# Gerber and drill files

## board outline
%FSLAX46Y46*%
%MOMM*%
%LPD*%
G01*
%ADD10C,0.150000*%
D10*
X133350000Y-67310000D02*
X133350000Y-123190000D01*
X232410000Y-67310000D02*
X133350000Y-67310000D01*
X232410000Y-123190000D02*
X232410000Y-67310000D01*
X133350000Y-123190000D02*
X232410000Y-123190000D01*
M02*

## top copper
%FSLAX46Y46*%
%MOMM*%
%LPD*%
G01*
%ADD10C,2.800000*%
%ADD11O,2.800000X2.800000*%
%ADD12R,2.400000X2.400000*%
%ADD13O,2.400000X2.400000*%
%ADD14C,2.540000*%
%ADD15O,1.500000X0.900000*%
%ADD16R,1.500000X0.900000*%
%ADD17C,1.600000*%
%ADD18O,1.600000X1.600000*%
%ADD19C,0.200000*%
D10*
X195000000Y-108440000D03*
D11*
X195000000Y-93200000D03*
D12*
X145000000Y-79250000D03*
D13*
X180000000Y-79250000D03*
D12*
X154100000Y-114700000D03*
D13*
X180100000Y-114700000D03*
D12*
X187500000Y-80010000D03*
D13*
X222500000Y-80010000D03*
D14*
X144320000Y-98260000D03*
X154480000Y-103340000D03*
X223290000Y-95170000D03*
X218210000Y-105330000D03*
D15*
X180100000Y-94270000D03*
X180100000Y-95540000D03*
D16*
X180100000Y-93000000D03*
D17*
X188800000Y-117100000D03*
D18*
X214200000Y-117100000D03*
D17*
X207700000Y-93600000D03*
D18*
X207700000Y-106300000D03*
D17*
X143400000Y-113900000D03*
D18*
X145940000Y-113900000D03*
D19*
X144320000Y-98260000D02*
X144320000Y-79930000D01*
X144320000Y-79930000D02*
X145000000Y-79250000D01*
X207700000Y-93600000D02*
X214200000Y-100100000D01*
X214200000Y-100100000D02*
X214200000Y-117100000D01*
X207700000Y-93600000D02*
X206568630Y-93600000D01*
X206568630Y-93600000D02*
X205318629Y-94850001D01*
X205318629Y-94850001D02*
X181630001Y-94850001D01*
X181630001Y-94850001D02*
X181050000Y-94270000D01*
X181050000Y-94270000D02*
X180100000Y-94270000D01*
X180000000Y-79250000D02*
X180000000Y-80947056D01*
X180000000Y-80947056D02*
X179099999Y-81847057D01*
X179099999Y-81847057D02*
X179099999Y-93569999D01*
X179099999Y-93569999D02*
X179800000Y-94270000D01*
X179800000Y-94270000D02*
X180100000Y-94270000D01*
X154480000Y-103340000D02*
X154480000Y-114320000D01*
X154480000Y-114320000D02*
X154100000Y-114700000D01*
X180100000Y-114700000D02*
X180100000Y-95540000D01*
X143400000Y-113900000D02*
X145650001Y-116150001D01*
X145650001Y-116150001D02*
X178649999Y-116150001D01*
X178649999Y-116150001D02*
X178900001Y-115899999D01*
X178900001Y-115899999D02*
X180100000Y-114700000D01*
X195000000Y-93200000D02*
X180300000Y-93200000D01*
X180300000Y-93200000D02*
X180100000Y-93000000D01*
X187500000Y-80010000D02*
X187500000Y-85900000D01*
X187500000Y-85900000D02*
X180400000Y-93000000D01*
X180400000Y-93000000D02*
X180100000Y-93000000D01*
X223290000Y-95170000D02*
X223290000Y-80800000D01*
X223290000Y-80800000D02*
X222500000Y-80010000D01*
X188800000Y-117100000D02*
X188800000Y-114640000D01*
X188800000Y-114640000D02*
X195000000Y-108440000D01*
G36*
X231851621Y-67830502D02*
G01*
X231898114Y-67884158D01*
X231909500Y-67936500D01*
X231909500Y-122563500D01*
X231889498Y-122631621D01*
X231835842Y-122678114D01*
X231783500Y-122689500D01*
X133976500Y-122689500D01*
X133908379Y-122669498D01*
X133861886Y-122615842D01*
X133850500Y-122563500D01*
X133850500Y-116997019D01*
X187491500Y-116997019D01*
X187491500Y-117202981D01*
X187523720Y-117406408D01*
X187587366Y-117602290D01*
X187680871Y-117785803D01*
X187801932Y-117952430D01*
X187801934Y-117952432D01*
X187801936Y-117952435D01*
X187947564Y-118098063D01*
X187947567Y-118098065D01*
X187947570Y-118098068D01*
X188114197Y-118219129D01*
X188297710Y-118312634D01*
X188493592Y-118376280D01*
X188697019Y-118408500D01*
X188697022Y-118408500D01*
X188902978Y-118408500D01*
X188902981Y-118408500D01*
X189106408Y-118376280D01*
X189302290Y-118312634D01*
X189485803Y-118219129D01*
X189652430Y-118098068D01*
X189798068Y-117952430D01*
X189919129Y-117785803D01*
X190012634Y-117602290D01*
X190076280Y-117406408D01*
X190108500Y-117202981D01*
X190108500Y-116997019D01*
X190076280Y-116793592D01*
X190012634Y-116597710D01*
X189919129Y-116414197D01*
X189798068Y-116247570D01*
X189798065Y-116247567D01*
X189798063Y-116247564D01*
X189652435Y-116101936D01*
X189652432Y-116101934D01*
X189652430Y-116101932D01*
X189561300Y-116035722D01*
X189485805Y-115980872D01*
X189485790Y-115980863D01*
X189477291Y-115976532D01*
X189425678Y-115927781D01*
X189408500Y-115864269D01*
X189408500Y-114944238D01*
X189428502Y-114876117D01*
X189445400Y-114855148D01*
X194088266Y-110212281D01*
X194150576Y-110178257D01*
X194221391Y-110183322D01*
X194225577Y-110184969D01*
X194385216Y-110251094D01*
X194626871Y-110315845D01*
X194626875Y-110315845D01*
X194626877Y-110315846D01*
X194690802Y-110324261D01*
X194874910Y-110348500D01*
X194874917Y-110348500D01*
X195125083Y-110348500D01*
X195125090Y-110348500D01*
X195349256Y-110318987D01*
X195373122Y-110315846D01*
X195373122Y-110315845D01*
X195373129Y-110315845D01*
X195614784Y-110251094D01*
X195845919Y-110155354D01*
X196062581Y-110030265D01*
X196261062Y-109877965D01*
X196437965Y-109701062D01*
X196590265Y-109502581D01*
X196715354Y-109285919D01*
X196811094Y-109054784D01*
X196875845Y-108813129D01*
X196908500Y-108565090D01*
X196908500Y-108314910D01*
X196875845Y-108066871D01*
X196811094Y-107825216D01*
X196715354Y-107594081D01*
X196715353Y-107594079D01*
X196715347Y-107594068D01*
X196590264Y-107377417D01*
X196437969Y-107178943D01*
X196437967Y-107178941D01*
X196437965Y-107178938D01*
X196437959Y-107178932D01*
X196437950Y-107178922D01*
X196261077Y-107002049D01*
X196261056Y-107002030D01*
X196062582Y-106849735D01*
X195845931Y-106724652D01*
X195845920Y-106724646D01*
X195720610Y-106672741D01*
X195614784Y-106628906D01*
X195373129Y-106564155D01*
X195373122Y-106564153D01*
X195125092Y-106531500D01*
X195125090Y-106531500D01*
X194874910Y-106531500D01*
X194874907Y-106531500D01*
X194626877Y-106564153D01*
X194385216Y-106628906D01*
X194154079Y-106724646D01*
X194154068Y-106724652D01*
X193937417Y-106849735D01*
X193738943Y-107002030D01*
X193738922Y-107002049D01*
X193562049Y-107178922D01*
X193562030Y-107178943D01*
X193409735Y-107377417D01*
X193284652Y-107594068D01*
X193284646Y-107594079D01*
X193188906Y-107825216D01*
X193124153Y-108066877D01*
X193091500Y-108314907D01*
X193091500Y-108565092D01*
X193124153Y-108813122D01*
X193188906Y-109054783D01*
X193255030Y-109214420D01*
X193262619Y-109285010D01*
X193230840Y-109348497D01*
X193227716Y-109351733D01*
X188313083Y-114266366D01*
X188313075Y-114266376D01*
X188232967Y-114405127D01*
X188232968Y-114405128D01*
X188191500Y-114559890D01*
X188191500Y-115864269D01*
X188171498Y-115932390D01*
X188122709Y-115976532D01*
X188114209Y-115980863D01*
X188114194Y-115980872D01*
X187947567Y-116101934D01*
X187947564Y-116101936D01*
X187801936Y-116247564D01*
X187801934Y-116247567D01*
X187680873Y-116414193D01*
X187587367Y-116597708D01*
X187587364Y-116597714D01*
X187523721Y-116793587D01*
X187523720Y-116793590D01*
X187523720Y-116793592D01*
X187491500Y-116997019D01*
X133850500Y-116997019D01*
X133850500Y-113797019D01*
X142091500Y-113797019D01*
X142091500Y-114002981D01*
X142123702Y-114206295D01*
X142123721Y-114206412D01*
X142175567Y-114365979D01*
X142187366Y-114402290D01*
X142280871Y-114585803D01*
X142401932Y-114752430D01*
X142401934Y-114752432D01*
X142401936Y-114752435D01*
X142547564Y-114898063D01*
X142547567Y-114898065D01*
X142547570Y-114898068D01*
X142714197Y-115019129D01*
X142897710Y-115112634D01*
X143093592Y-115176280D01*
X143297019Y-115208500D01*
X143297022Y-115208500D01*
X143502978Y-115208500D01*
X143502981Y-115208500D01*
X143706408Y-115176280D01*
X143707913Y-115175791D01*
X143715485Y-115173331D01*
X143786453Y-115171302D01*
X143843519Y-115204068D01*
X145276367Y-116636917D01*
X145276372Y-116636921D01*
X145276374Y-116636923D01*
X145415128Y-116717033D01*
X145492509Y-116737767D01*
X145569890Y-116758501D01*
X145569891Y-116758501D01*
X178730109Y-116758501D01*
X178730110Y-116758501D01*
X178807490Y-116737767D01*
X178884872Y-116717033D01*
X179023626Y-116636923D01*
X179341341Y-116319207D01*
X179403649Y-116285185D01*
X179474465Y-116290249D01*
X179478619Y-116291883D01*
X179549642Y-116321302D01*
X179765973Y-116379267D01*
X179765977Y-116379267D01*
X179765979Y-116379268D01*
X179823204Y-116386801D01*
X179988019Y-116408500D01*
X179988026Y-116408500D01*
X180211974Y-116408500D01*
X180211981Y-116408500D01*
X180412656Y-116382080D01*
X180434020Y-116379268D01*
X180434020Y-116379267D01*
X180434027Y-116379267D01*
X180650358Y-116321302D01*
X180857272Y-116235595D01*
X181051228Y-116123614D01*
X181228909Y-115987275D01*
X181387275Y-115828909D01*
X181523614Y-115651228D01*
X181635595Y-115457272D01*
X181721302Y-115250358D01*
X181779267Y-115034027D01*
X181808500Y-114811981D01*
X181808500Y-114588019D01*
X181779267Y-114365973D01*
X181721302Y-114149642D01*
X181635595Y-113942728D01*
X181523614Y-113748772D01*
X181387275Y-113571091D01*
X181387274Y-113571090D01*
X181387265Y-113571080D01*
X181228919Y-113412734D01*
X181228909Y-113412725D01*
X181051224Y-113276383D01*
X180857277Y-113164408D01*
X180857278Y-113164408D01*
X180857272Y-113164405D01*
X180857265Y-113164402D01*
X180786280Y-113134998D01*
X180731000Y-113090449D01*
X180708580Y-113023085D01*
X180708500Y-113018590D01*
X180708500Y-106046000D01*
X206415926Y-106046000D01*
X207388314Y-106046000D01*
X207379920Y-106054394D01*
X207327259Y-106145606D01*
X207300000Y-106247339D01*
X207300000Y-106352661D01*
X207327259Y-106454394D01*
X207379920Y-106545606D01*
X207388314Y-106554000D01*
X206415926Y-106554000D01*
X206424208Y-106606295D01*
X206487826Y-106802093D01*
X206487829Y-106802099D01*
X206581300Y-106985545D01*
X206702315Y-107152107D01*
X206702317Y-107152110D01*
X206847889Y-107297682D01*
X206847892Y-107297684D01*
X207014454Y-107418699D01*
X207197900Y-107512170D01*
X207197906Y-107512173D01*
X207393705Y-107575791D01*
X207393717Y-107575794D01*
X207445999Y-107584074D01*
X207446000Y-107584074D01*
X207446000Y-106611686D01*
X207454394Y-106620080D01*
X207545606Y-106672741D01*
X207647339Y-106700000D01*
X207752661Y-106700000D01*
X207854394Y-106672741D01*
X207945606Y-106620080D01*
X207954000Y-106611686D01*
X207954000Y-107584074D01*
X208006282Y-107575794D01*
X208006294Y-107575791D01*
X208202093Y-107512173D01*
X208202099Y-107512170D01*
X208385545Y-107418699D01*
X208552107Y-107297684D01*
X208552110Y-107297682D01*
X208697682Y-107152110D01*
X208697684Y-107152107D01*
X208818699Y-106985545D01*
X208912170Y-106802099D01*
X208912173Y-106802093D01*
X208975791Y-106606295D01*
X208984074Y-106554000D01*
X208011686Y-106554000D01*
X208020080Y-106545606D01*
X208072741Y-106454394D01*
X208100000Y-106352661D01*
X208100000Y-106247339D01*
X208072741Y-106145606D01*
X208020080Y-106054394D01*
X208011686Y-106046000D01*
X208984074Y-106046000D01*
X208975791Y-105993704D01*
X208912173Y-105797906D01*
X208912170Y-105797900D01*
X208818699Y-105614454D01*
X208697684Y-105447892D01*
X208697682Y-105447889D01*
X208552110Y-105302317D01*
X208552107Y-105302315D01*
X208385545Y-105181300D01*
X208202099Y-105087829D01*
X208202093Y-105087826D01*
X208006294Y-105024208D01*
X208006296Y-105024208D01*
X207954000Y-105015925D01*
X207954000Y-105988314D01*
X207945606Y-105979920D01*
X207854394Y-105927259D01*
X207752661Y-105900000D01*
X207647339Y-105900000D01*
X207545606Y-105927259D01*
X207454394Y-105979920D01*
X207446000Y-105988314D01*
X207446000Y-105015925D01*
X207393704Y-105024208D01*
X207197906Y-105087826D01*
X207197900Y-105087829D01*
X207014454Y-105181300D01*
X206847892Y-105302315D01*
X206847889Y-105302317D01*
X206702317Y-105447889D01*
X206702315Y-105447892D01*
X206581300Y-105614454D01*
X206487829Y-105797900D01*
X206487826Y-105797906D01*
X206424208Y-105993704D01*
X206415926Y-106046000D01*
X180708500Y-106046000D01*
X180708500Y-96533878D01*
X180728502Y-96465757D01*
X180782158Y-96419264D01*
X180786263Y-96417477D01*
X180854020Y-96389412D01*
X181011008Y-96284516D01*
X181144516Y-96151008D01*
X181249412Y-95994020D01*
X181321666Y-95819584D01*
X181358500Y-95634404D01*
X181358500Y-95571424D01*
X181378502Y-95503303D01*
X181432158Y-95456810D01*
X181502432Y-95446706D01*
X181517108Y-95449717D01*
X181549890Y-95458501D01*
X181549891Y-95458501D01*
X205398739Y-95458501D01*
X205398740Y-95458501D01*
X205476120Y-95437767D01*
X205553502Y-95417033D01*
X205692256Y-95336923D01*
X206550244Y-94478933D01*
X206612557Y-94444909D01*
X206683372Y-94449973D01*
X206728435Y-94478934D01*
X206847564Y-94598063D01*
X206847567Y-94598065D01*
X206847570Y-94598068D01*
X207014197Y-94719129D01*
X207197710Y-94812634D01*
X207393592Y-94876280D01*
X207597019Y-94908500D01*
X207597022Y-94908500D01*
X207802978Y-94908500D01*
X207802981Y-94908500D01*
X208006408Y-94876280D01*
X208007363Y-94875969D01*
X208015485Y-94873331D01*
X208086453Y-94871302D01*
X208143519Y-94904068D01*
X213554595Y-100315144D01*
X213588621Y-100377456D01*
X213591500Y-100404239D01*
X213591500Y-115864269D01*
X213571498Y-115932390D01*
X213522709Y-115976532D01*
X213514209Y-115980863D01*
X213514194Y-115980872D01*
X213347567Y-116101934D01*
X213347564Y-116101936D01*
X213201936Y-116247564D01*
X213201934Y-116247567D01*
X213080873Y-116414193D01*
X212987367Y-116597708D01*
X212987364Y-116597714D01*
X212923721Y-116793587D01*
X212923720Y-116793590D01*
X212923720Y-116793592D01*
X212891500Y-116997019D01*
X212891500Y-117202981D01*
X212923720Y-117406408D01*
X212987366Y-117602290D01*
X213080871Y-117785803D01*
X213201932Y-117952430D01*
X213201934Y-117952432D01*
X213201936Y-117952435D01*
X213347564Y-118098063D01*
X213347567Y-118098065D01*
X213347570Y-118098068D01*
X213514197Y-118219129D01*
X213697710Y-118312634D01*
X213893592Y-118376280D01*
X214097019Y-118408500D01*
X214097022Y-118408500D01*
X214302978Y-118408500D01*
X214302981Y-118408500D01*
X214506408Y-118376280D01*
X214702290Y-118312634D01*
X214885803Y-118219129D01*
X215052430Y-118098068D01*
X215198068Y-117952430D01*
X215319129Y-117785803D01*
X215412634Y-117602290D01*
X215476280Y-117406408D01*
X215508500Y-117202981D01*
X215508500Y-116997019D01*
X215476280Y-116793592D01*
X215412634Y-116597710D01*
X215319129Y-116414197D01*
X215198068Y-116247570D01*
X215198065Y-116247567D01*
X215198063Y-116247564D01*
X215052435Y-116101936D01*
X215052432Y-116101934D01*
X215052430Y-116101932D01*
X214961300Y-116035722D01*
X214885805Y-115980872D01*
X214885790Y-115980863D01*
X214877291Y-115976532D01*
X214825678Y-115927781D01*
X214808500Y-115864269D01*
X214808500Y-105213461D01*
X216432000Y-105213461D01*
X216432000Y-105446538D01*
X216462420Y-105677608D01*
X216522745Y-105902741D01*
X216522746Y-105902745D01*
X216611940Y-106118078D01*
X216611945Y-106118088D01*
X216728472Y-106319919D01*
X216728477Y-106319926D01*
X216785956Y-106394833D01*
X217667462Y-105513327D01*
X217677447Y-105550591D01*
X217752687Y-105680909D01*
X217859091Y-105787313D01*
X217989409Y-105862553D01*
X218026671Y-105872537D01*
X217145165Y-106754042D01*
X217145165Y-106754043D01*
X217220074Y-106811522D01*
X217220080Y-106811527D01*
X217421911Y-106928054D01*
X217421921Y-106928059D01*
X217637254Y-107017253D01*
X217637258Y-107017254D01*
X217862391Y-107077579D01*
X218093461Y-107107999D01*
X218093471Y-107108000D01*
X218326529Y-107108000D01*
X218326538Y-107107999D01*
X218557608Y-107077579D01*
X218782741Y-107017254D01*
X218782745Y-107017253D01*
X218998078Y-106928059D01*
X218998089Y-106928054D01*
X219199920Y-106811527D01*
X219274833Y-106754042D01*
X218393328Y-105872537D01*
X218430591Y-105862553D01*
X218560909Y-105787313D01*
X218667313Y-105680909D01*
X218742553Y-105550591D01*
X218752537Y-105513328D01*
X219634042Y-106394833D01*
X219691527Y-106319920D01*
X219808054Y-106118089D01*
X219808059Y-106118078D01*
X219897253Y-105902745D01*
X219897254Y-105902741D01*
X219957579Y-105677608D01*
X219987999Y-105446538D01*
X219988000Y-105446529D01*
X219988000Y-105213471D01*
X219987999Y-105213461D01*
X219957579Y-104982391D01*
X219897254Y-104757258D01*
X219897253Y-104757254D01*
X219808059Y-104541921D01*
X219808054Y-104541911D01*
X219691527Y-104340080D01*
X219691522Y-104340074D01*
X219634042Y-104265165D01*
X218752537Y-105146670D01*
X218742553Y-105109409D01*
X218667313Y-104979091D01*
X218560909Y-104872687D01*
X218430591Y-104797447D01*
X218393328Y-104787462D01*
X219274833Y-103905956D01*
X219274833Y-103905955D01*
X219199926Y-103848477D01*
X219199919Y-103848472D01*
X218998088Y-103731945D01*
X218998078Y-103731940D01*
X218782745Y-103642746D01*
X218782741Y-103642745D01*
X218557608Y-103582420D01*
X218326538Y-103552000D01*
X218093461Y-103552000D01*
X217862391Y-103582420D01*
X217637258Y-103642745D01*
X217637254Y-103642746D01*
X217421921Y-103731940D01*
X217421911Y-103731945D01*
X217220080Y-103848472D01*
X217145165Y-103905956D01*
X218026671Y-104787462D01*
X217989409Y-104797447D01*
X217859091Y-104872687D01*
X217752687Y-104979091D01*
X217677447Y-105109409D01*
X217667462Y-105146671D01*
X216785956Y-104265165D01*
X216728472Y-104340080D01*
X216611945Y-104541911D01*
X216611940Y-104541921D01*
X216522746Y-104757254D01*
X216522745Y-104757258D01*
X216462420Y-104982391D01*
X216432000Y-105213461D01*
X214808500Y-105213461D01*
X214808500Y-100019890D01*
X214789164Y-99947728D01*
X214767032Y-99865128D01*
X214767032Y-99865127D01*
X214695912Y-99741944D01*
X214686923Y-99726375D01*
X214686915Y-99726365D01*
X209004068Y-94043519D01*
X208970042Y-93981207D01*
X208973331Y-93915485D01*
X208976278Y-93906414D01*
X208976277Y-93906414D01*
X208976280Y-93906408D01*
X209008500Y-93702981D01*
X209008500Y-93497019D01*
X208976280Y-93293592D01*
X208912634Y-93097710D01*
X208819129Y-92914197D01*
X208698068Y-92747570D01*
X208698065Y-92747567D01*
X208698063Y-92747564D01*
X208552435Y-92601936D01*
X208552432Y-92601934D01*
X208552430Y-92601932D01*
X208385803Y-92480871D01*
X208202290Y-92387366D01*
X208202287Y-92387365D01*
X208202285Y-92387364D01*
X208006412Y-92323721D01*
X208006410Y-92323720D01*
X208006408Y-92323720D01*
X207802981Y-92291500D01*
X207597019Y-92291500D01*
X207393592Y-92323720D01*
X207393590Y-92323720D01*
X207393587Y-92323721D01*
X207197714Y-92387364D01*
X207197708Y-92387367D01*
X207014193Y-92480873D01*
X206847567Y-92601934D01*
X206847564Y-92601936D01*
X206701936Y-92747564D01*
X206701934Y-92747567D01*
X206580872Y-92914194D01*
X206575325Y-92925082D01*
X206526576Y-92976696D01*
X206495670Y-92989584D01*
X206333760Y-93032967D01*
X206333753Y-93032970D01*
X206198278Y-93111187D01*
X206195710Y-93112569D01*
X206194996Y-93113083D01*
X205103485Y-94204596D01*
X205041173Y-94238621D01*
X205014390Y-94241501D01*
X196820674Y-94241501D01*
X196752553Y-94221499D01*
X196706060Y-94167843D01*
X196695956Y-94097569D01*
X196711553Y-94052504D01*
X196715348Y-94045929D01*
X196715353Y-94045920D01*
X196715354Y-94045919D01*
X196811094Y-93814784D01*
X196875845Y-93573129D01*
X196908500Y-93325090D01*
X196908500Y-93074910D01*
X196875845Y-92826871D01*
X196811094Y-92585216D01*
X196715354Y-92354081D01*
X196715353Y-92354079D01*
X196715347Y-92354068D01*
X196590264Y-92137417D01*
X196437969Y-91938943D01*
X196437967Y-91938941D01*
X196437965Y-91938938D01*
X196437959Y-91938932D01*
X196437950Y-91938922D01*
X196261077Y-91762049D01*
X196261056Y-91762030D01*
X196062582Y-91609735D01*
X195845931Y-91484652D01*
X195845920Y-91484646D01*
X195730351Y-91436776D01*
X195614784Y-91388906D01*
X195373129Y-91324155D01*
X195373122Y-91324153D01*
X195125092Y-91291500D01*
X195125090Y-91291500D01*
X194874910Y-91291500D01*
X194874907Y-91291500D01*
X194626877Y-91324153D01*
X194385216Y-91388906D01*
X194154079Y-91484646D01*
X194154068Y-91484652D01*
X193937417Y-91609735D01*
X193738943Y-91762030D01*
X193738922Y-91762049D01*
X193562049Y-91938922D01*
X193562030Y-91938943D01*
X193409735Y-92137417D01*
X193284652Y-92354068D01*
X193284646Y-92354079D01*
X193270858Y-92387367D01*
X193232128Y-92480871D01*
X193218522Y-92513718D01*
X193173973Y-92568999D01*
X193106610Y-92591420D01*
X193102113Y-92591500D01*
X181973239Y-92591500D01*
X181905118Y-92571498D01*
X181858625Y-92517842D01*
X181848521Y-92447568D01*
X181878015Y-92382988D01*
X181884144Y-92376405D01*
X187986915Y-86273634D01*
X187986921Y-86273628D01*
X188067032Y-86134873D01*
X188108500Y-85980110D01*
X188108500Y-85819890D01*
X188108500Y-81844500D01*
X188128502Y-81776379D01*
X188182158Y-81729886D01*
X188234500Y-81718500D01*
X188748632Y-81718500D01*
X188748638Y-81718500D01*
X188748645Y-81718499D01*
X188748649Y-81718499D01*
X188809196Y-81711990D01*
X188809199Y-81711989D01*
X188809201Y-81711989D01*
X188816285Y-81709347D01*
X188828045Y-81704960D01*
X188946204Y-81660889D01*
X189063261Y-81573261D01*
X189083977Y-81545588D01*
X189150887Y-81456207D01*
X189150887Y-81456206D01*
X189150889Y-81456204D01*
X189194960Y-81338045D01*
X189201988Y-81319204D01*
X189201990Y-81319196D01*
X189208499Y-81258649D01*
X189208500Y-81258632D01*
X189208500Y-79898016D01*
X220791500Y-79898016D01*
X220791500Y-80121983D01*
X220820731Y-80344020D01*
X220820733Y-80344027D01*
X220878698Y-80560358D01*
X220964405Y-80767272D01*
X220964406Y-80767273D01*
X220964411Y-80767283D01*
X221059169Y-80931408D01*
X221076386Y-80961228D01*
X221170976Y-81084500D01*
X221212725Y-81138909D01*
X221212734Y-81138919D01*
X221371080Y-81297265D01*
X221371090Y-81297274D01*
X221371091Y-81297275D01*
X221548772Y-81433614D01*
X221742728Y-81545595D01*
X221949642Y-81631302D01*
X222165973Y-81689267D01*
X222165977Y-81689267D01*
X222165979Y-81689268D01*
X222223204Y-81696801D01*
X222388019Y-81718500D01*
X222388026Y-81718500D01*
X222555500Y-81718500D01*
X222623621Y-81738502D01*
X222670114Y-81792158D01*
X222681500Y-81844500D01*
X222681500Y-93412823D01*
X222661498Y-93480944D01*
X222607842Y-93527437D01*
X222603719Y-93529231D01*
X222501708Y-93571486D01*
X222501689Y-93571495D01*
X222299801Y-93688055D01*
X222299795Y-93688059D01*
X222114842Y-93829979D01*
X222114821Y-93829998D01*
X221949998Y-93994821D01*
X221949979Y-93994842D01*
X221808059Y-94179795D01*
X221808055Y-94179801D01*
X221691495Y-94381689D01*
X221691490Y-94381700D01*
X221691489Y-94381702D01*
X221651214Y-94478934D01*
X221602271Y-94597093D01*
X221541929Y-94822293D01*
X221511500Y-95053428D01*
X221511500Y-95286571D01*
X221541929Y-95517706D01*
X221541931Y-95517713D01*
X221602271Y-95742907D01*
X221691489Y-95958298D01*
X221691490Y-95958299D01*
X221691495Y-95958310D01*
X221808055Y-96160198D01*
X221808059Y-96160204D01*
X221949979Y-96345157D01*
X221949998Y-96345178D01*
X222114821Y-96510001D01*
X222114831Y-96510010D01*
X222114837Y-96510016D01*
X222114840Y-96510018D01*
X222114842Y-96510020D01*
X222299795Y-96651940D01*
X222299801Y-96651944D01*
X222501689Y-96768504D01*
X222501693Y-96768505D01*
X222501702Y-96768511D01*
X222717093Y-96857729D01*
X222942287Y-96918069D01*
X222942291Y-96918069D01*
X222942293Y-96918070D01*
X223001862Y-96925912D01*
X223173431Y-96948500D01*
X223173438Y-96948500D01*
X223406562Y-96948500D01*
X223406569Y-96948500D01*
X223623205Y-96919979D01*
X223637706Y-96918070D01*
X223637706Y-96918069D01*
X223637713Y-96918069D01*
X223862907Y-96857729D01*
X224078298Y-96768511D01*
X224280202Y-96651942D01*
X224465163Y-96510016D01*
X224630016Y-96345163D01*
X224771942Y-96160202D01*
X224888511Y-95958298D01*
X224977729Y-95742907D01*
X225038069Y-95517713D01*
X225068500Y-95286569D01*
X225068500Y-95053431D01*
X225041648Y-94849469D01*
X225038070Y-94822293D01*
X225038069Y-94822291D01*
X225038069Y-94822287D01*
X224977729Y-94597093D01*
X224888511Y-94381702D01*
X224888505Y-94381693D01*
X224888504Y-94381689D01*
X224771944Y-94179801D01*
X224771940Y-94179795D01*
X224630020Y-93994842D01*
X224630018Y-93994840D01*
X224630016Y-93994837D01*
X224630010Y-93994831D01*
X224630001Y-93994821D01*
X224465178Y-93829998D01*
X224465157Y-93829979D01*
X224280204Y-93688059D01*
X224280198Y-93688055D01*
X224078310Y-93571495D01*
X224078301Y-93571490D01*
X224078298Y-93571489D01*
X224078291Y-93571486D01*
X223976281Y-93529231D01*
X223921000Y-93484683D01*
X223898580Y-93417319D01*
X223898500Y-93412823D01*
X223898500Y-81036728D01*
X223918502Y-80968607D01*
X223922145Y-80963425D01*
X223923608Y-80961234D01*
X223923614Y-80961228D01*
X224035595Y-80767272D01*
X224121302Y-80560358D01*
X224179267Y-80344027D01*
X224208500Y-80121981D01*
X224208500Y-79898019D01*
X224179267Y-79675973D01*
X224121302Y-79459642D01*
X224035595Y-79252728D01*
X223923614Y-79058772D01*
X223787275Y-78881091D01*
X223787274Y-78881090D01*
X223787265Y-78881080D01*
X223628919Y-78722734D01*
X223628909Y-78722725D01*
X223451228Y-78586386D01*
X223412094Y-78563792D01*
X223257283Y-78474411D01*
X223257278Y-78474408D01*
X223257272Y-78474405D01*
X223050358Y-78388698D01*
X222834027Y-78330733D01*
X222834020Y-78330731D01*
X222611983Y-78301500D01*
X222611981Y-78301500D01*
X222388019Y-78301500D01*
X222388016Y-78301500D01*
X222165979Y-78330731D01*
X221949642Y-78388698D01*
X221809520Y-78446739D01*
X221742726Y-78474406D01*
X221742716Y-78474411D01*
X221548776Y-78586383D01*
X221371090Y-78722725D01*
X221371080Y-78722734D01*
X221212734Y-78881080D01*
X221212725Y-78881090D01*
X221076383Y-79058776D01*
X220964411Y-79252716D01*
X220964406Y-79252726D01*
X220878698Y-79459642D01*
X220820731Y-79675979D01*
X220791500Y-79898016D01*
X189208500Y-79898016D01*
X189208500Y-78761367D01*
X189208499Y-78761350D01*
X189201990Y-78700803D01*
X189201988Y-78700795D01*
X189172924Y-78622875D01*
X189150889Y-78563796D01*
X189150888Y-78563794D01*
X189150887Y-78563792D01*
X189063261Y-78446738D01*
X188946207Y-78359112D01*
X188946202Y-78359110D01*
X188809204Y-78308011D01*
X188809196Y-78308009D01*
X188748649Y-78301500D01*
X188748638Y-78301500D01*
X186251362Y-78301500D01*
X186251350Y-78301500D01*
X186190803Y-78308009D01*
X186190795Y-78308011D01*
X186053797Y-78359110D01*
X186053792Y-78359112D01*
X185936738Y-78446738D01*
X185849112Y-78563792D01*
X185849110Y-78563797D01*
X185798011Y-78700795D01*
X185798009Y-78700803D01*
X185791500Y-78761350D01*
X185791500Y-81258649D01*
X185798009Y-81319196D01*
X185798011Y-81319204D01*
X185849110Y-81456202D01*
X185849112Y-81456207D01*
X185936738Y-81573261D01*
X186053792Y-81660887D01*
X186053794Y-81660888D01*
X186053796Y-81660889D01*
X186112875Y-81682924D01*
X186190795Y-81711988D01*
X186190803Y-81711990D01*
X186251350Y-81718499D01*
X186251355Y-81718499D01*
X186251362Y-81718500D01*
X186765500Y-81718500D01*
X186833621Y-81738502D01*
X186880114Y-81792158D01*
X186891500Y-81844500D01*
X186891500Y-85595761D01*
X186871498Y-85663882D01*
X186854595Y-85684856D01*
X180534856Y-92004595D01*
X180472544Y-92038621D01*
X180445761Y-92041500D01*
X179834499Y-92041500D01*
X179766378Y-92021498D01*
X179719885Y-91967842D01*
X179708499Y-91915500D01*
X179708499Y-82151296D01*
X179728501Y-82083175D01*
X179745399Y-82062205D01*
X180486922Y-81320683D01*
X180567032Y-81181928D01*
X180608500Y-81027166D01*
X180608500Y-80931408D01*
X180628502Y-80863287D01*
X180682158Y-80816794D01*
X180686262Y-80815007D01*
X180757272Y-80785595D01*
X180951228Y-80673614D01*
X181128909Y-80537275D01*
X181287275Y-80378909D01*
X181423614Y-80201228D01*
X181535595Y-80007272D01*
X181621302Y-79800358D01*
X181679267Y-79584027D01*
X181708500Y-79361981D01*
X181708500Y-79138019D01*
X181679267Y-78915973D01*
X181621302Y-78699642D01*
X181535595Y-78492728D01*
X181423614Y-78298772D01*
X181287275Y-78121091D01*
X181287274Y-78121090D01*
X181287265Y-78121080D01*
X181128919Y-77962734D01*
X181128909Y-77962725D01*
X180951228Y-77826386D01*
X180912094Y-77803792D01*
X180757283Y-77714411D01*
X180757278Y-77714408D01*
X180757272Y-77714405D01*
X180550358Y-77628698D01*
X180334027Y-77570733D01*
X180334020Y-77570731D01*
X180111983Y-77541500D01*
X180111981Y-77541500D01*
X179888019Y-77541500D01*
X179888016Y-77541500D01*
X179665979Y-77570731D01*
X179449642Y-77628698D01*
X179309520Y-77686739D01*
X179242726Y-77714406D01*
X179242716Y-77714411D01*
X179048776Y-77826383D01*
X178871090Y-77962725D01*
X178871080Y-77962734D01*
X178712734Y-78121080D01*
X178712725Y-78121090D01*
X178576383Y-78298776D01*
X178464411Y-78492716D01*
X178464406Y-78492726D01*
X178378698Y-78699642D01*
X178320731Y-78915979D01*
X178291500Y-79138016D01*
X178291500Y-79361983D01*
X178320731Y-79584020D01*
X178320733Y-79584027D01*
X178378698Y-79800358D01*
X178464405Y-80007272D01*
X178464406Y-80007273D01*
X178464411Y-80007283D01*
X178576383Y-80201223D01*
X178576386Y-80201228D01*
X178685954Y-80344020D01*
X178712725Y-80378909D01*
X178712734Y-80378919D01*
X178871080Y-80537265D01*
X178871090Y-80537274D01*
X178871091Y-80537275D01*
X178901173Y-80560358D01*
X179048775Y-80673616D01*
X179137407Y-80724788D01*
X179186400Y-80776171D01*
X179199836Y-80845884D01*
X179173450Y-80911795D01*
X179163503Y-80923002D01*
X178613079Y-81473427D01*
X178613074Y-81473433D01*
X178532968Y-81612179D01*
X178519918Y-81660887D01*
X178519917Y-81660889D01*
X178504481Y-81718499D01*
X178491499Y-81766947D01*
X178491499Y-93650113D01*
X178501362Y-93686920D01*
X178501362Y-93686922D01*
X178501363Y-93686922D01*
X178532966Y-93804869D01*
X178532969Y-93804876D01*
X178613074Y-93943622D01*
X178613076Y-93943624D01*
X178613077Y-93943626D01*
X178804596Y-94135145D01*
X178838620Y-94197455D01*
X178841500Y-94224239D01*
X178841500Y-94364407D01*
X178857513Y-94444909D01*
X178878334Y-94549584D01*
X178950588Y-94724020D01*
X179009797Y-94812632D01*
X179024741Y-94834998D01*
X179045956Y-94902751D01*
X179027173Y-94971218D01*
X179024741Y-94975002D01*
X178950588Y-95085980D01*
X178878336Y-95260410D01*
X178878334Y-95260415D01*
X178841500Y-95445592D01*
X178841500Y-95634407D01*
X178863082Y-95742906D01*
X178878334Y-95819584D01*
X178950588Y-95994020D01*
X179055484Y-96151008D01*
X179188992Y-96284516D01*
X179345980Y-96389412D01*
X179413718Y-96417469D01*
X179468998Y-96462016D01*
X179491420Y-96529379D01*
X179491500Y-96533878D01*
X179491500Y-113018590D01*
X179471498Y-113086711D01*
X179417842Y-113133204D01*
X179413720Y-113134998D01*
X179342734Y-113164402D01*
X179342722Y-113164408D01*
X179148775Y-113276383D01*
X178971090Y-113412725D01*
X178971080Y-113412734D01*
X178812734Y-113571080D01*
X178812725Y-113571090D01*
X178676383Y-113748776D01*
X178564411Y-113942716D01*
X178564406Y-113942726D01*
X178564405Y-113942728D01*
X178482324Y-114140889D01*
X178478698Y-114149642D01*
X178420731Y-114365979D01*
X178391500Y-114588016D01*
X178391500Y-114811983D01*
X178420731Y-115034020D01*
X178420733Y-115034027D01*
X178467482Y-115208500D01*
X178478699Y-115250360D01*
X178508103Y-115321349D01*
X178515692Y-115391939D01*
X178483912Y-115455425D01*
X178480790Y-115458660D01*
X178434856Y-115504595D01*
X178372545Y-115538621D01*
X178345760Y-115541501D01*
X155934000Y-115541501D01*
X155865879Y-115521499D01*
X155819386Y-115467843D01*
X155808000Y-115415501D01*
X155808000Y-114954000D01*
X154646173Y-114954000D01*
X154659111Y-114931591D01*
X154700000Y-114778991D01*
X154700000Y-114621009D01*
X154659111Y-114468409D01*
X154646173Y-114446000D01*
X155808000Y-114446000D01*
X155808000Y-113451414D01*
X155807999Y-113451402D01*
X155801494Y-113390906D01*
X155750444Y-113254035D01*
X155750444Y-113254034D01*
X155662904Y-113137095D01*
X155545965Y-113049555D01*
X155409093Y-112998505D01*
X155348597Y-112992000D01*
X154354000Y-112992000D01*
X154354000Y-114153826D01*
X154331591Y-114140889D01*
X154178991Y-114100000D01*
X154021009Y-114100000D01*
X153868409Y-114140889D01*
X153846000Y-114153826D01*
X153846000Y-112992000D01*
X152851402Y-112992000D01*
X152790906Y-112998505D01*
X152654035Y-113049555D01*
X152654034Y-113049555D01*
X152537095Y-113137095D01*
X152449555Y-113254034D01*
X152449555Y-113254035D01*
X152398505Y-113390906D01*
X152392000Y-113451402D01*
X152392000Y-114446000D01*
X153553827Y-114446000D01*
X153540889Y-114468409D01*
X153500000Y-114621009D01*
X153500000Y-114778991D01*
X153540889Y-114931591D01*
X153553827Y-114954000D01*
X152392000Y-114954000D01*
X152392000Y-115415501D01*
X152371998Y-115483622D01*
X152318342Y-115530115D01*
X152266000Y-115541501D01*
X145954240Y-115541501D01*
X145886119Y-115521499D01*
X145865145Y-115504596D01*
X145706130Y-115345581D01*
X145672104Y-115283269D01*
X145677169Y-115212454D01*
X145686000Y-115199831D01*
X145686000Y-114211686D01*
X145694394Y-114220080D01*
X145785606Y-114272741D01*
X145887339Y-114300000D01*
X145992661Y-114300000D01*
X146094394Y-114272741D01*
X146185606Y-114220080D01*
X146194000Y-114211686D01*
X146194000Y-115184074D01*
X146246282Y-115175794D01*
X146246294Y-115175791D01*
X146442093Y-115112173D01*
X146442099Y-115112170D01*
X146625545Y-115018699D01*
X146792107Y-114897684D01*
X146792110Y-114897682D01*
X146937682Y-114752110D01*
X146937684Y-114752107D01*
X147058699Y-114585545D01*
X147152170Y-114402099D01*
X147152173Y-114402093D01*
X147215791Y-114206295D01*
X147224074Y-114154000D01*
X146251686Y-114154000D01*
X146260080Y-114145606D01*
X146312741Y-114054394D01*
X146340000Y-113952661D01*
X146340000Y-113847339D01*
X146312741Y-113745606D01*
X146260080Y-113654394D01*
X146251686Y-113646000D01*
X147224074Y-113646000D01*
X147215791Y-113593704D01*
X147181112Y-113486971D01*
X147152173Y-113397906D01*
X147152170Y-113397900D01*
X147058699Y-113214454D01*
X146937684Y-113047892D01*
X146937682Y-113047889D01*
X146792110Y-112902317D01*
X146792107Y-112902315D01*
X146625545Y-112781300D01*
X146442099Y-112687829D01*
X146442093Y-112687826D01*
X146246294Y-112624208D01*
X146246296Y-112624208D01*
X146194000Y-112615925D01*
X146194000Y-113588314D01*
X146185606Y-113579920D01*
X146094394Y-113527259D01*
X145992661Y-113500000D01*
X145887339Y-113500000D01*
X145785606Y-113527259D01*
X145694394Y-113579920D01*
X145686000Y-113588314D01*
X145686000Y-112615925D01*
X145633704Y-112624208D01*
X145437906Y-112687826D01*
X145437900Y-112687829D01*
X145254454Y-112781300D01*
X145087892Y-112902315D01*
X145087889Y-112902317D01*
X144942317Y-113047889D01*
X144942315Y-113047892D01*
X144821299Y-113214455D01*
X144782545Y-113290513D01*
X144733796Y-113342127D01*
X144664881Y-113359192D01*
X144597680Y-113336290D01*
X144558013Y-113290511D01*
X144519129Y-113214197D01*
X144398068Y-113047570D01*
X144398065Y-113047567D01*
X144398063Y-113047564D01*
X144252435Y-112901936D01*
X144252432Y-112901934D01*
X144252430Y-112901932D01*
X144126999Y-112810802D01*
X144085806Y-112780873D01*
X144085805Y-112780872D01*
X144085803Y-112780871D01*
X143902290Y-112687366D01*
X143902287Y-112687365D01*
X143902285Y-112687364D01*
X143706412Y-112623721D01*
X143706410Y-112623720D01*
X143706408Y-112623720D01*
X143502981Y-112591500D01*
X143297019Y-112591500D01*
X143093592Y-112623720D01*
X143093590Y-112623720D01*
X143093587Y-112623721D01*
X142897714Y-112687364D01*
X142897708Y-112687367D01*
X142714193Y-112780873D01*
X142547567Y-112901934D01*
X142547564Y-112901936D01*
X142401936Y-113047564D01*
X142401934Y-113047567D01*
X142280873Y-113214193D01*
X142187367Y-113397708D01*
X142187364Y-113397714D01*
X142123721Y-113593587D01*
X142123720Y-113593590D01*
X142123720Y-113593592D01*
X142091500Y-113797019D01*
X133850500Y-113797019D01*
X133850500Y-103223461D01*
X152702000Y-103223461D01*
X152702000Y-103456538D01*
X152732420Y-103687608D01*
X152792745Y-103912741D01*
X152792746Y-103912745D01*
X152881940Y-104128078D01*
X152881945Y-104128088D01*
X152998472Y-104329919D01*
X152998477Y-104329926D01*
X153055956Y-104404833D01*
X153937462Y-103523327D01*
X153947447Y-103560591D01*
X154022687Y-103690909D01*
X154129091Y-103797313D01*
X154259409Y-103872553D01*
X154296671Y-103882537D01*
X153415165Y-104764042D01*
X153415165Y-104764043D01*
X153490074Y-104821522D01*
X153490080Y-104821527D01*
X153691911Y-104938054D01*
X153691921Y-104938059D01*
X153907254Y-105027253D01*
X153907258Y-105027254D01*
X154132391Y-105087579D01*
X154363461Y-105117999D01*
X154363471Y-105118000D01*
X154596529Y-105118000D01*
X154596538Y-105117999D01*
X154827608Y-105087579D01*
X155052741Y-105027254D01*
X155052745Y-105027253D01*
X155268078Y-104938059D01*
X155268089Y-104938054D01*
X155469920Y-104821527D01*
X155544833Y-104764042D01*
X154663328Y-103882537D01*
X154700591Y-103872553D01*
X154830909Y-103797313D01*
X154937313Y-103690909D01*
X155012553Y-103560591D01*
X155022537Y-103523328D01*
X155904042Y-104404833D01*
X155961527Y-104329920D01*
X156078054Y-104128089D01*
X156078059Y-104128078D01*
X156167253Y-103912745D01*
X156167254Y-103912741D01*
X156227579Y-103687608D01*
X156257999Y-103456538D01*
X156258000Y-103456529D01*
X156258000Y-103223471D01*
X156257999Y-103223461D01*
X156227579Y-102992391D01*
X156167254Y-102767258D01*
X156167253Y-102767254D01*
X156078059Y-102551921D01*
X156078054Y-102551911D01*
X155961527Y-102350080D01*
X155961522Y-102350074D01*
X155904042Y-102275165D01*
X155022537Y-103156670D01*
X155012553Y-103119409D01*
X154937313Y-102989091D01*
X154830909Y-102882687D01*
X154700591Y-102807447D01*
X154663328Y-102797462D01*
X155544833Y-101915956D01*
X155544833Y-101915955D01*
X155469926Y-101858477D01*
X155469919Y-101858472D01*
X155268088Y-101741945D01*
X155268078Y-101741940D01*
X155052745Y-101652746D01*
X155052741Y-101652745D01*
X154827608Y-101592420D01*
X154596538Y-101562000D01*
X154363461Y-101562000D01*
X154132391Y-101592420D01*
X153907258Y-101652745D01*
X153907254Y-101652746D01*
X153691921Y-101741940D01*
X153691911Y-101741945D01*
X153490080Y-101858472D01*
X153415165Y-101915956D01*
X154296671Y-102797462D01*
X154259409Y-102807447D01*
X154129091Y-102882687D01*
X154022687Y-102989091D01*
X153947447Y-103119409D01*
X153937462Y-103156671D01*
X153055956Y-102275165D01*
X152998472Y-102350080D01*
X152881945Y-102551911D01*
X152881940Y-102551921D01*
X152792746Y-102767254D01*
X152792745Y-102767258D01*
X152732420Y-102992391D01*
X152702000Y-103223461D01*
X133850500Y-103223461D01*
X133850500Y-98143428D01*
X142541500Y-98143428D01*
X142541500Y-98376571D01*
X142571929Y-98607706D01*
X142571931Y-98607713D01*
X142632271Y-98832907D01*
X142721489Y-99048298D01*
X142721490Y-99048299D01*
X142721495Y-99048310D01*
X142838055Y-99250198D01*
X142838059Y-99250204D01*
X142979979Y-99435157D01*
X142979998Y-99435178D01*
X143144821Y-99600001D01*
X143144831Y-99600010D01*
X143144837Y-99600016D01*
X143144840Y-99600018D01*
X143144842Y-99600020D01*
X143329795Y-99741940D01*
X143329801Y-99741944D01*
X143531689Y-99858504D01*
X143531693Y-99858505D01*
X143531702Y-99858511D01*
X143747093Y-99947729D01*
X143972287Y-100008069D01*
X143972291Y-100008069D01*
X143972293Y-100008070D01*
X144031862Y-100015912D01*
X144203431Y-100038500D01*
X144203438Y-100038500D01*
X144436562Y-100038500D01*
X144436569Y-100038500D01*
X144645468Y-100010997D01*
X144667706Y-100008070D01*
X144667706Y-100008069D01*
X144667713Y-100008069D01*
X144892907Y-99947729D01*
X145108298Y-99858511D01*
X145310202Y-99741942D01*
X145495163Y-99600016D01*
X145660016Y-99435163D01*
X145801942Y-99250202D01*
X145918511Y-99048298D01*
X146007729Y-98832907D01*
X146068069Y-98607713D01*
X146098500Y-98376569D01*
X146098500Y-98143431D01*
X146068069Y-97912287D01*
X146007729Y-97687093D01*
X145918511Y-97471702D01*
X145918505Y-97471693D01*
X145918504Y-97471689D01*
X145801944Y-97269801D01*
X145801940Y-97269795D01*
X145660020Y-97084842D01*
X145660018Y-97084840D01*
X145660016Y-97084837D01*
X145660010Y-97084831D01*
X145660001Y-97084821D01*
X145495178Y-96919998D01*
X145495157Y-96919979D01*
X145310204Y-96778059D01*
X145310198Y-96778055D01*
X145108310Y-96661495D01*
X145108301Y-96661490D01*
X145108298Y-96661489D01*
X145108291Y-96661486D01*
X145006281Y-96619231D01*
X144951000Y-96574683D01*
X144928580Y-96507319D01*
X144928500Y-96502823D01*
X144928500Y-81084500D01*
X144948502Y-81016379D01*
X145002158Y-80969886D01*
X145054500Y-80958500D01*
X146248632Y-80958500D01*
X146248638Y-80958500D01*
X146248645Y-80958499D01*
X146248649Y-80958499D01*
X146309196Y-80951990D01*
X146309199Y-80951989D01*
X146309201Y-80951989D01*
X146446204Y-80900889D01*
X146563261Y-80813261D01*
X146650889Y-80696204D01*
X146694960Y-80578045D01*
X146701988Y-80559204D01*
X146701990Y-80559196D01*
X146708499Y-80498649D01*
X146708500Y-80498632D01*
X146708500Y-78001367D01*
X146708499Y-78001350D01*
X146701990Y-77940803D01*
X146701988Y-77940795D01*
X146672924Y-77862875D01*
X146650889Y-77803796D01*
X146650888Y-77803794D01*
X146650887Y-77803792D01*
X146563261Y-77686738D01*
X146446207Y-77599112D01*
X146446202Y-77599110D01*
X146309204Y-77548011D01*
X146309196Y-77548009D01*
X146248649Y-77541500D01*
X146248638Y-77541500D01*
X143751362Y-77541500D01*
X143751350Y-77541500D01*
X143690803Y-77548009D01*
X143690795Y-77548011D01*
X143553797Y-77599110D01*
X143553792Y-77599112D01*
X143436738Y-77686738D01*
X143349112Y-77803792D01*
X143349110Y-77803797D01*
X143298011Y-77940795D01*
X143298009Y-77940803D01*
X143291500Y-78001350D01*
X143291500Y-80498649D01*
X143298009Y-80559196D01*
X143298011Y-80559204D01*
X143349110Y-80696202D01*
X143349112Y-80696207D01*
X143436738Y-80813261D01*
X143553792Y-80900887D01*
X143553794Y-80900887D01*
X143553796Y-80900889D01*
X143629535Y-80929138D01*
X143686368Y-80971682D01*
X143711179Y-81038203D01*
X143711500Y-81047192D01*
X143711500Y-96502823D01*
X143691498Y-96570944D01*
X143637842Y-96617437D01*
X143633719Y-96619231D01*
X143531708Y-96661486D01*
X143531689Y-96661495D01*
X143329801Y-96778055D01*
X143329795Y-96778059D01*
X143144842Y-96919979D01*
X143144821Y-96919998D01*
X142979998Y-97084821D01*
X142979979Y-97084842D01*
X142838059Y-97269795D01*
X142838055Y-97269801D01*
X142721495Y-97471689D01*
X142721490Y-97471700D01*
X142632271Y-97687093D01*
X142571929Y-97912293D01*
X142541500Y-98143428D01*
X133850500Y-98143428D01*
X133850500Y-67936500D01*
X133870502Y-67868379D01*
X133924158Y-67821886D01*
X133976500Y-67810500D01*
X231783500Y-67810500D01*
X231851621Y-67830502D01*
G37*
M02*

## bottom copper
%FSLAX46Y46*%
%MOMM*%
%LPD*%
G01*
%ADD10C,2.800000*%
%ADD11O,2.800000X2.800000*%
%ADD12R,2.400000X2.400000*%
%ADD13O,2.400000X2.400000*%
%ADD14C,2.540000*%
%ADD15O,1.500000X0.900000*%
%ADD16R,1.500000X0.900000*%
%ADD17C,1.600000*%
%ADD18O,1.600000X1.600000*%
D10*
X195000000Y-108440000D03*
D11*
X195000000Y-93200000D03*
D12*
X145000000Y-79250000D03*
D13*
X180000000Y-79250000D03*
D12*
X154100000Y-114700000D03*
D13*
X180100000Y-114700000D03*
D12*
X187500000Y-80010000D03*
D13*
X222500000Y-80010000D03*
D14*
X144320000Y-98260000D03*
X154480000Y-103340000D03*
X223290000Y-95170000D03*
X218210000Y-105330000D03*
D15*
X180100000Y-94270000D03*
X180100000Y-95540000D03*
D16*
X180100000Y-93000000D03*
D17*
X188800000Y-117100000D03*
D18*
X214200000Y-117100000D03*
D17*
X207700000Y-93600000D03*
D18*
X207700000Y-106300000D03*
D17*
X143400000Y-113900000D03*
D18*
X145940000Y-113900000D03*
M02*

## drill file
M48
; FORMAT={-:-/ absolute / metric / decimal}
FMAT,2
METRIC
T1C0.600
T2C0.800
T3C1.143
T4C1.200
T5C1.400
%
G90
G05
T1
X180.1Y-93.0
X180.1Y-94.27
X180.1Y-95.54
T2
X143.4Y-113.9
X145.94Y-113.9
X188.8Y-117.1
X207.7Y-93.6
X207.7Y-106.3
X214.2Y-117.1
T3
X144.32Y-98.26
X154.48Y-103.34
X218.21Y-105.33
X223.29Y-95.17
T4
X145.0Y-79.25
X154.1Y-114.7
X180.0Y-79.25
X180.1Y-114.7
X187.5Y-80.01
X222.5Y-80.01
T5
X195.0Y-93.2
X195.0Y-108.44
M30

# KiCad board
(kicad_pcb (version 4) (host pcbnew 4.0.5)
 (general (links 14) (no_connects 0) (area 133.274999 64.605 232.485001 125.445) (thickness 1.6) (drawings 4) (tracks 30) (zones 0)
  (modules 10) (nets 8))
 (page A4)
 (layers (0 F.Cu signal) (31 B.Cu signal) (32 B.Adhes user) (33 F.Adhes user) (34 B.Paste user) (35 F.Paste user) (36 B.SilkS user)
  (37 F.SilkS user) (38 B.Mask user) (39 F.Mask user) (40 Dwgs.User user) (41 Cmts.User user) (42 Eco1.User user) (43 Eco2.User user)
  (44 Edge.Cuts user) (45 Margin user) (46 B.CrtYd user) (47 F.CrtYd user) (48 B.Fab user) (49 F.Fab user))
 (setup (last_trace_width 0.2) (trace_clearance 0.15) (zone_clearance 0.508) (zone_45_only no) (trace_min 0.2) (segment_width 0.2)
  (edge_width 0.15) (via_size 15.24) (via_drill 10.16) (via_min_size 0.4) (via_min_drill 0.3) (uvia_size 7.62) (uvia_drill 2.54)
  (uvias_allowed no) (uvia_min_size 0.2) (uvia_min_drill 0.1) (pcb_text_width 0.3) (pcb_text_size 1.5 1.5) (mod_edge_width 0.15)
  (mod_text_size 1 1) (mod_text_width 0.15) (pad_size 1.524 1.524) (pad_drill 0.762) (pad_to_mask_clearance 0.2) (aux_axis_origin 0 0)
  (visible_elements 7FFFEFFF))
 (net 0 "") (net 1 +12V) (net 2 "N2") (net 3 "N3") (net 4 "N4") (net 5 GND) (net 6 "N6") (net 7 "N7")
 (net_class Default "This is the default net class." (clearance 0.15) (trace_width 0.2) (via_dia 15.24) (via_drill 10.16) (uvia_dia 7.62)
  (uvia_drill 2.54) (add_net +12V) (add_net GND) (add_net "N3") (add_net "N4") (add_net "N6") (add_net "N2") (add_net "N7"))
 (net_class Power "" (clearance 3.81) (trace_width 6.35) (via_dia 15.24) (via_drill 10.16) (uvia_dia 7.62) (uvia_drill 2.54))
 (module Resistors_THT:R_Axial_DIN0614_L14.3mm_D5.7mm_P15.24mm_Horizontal (layer F.Cu) (at 195 108.44 90)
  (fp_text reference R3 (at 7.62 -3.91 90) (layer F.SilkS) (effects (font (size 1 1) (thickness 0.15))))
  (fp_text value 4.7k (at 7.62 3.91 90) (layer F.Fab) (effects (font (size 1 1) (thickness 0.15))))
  (pad 1 thru_hole circle (at 0 0 90) (size 2.8 2.8) (drill 1.4) (layers *.Cu *.Mask) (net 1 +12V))
  (pad 2 thru_hole oval (at 15.24 0 90) (size 2.8 2.8) (drill 1.4) (layers *.Cu *.Mask) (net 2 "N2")))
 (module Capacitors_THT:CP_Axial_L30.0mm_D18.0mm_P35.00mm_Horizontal (layer F.Cu) (at 145 79.25)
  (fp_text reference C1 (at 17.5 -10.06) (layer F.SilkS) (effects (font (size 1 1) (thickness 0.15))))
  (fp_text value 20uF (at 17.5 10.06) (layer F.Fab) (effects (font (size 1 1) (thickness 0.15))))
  (pad 1 thru_hole rect (at 0 0) (size 2.4 2.4) (drill 1.2) (layers *.Cu *.Mask) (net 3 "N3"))
  (pad 2 thru_hole oval (at 35 0) (size 2.4 2.4) (drill 1.2) (layers *.Cu *.Mask) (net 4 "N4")))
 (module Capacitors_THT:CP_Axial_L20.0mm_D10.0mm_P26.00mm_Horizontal (layer F.Cu) (at 154.1 114.7)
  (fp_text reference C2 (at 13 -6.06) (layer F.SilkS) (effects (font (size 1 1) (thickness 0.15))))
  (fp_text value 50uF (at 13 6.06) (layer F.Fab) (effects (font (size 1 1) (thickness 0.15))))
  (pad 1 thru_hole rect (at 0 0) (size 2.4 2.4) (drill 1.2) (layers *.Cu *.Mask) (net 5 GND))
  (pad 2 thru_hole oval (at 26 0) (size 2.4 2.4) (drill 1.2) (layers *.Cu *.Mask) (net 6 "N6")))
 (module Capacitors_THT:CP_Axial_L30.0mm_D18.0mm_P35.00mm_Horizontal (layer F.Cu) (at 187.5 80.01)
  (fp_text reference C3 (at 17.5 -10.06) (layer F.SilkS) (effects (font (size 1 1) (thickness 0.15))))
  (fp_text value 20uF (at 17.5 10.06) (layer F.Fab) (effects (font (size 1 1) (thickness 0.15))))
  (pad 1 thru_hole rect (at 0 0) (size 2.4 2.4) (drill 1.2) (layers *.Cu *.Mask) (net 2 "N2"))
  (pad 2 thru_hole oval (at 35 0) (size 2.4 2.4) (drill 1.2) (layers *.Cu *.Mask) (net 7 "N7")))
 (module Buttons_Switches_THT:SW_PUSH (layer F.Cu) (at 149.4 100.8)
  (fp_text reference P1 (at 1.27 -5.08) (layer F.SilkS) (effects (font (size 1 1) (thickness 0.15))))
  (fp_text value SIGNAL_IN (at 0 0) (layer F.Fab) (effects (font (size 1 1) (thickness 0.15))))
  (pad 1 thru_hole circle (at -5.08 -2.54) (size 2.54 2.54) (drill 1.143) (layers *.Cu *.Mask) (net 3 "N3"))
  (pad 2 thru_hole circle (at 5.08 2.54) (size 2.54 2.54) (drill 1.143) (layers *.Cu *.Mask) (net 5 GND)))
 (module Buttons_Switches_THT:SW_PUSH (layer F.Cu) (at 220.75 100.25 270)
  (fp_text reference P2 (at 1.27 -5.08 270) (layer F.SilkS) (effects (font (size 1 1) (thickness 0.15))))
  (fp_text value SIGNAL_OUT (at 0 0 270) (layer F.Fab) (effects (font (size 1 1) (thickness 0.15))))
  (pad 1 thru_hole circle (at -5.08 -2.54 270) (size 2.54 2.54) (drill 1.143) (layers *.Cu *.Mask) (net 7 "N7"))
  (pad 2 thru_hole circle (at 5.08 2.54 270) (size 2.54 2.54) (drill 1.143) (layers *.Cu *.Mask) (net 5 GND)))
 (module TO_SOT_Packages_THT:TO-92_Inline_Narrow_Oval (layer F.Cu) (at 180.1 93 270)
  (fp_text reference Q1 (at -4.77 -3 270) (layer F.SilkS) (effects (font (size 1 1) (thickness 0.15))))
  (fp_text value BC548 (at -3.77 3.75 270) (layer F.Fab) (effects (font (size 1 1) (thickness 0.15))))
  (pad 2 thru_hole oval (at 1.27 0 90) (size 0.9 1.5) (drill 0.6) (layers *.Cu *.Mask) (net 4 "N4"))
  (pad 3 thru_hole oval (at 2.54 0 90) (size 0.9 1.5) (drill 0.6) (layers *.Cu *.Mask) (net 6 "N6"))
  (pad 1 thru_hole rect (at 0 0 90) (size 0.9 1.5) (drill 0.6) (layers *.Cu *.Mask) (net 2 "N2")))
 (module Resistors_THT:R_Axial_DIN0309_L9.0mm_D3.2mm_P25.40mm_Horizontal (layer F.Cu) (at 188.8 117.1)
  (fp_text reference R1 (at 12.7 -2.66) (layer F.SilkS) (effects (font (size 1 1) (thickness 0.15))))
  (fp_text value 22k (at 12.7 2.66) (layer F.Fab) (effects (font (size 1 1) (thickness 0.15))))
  (pad 1 thru_hole circle (at 0 0) (size 1.6 1.6) (drill 0.8) (layers *.Cu *.Mask) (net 1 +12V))
  (pad 2 thru_hole oval (at 25.4 0) (size 1.6 1.6) (drill 0.8) (layers *.Cu *.Mask) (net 4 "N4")))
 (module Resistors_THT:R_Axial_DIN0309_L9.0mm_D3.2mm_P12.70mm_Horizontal (layer F.Cu) (at 207.7 93.6 270)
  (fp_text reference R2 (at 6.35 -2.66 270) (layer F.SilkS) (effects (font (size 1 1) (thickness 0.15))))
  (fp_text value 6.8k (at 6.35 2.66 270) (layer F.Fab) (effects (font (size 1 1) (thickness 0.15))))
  (pad 1 thru_hole circle (at 0 0 270) (size 1.6 1.6) (drill 0.8) (layers *.Cu *.Mask) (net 4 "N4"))
  (pad 2 thru_hole oval (at 12.7 0 270) (size 1.6 1.6) (drill 0.8) (layers *.Cu *.Mask) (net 5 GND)))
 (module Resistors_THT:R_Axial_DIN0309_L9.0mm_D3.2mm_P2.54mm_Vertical (layer F.Cu) (at 143.4 113.9)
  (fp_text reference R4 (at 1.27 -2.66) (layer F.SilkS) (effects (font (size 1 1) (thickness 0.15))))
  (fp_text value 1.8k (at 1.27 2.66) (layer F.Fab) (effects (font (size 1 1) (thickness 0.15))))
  (pad 1 thru_hole circle (at 0 0) (size 1.6 1.6) (drill 0.8) (layers *.Cu *.Mask) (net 6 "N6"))
  (pad 2 thru_hole oval (at 2.54 0) (size 1.6 1.6) (drill 0.8) (layers *.Cu *.Mask) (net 5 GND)))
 (gr_line (start 133.35 67.31) (end 133.35 123.19) (layer Edge.Cuts) (width 0.15))
 (gr_line (start 232.41 67.31) (end 133.35 67.31) (layer Edge.Cuts) (width 0.15))
 (gr_line (start 232.41 123.19) (end 232.41 67.31) (layer Edge.Cuts) (width 0.15))
 (gr_line (start 133.35 123.19) (end 232.41 123.19) (layer Edge.Cuts) (width 0.15))
 (segment (start 144.32 98.26) (end 144.32 79.93) (width 0.2) (layer F.Cu) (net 3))
 (segment (start 144.32 79.93) (end 145 79.25) (width 0.2) (layer F.Cu) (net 3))
 (segment (start 207.7 93.6) (end 214.2 100.1) (width 0.2) (layer F.Cu) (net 4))
 (segment (start 214.2 100.1) (end 214.2 117.1) (width 0.2) (layer F.Cu) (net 4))
 (segment (start 207.7 93.6) (end 206.56863 93.6) (width 0.2) (layer F.Cu) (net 4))
 (segment (start 206.56863 93.6) (end 205.318629 94.850001) (width 0.2) (layer F.Cu) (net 4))
 (segment (start 205.318629 94.850001) (end 181.630001 94.850001) (width 0.2) (layer F.Cu) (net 4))
 (segment (start 181.630001 94.850001) (end 181.05 94.27) (width 0.2) (layer F.Cu) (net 4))
 (segment (start 181.05 94.27) (end 180.1 94.27) (width 0.2) (layer F.Cu) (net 4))
 (segment (start 180 79.25) (end 180 80.947056) (width 0.2) (layer F.Cu) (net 4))
 (segment (start 180 80.947056) (end 179.099999 81.847057) (width 0.2) (layer F.Cu) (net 4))
 (segment (start 179.099999 81.847057) (end 179.099999 93.569999) (width 0.2) (layer F.Cu) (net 4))
 (segment (start 179.099999 93.569999) (end 179.8 94.27) (width 0.2) (layer F.Cu) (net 4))
 (segment (start 179.8 94.27) (end 180.1 94.27) (width 0.2) (layer F.Cu) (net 4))
 (segment (start 154.48 103.34) (end 154.48 114.32) (width 0.2) (layer F.Cu) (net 5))
 (segment (start 154.48 114.32) (end 154.1 114.7) (width 0.2) (layer F.Cu) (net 5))
 (segment (start 180.1 114.7) (end 180.1 95.54) (width 0.2) (layer F.Cu) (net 6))
 (segment (start 143.4 113.9) (end 145.650001 116.150001) (width 0.2) (layer F.Cu) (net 6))
 (segment (start 145.650001 116.150001) (end 178.649999 116.150001) (width 0.2) (layer F.Cu) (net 6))
 (segment (start 178.649999 116.150001) (end 178.900001 115.899999) (width 0.2) (layer F.Cu) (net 6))
 (segment (start 178.900001 115.899999) (end 180.1 114.7) (width 0.2) (layer F.Cu) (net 6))
 (segment (start 195 93.2) (end 180.3 93.2) (width 0.2) (layer F.Cu) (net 2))
 (segment (start 180.3 93.2) (end 180.1 93) (width 0.2) (layer F.Cu) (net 2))
 (segment (start 187.5 80.01) (end 187.5 85.9) (width 0.2) (layer F.Cu) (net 2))
 (segment (start 187.5 85.9) (end 180.4 93) (width 0.2) (layer F.Cu) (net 2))
 (segment (start 180.4 93) (end 180.1 93) (width 0.2) (layer F.Cu) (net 2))
 (segment (start 223.29 95.17) (end 223.29 80.8) (width 0.2) (layer F.Cu) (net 7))
 (segment (start 223.29 80.8) (end 222.5 80.01) (width 0.2) (layer F.Cu) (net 7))
 (segment (start 188.8 117.1) (end 188.8 114.64) (width 0.2) (layer F.Cu) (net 1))
 (segment (start 188.8 114.64) (end 195 108.44) (width 0.2) (layer F.Cu) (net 1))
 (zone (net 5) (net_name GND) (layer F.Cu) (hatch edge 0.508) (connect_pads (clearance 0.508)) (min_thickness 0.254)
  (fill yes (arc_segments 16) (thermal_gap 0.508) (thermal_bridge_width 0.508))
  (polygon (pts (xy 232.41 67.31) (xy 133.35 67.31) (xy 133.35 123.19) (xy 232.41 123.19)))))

